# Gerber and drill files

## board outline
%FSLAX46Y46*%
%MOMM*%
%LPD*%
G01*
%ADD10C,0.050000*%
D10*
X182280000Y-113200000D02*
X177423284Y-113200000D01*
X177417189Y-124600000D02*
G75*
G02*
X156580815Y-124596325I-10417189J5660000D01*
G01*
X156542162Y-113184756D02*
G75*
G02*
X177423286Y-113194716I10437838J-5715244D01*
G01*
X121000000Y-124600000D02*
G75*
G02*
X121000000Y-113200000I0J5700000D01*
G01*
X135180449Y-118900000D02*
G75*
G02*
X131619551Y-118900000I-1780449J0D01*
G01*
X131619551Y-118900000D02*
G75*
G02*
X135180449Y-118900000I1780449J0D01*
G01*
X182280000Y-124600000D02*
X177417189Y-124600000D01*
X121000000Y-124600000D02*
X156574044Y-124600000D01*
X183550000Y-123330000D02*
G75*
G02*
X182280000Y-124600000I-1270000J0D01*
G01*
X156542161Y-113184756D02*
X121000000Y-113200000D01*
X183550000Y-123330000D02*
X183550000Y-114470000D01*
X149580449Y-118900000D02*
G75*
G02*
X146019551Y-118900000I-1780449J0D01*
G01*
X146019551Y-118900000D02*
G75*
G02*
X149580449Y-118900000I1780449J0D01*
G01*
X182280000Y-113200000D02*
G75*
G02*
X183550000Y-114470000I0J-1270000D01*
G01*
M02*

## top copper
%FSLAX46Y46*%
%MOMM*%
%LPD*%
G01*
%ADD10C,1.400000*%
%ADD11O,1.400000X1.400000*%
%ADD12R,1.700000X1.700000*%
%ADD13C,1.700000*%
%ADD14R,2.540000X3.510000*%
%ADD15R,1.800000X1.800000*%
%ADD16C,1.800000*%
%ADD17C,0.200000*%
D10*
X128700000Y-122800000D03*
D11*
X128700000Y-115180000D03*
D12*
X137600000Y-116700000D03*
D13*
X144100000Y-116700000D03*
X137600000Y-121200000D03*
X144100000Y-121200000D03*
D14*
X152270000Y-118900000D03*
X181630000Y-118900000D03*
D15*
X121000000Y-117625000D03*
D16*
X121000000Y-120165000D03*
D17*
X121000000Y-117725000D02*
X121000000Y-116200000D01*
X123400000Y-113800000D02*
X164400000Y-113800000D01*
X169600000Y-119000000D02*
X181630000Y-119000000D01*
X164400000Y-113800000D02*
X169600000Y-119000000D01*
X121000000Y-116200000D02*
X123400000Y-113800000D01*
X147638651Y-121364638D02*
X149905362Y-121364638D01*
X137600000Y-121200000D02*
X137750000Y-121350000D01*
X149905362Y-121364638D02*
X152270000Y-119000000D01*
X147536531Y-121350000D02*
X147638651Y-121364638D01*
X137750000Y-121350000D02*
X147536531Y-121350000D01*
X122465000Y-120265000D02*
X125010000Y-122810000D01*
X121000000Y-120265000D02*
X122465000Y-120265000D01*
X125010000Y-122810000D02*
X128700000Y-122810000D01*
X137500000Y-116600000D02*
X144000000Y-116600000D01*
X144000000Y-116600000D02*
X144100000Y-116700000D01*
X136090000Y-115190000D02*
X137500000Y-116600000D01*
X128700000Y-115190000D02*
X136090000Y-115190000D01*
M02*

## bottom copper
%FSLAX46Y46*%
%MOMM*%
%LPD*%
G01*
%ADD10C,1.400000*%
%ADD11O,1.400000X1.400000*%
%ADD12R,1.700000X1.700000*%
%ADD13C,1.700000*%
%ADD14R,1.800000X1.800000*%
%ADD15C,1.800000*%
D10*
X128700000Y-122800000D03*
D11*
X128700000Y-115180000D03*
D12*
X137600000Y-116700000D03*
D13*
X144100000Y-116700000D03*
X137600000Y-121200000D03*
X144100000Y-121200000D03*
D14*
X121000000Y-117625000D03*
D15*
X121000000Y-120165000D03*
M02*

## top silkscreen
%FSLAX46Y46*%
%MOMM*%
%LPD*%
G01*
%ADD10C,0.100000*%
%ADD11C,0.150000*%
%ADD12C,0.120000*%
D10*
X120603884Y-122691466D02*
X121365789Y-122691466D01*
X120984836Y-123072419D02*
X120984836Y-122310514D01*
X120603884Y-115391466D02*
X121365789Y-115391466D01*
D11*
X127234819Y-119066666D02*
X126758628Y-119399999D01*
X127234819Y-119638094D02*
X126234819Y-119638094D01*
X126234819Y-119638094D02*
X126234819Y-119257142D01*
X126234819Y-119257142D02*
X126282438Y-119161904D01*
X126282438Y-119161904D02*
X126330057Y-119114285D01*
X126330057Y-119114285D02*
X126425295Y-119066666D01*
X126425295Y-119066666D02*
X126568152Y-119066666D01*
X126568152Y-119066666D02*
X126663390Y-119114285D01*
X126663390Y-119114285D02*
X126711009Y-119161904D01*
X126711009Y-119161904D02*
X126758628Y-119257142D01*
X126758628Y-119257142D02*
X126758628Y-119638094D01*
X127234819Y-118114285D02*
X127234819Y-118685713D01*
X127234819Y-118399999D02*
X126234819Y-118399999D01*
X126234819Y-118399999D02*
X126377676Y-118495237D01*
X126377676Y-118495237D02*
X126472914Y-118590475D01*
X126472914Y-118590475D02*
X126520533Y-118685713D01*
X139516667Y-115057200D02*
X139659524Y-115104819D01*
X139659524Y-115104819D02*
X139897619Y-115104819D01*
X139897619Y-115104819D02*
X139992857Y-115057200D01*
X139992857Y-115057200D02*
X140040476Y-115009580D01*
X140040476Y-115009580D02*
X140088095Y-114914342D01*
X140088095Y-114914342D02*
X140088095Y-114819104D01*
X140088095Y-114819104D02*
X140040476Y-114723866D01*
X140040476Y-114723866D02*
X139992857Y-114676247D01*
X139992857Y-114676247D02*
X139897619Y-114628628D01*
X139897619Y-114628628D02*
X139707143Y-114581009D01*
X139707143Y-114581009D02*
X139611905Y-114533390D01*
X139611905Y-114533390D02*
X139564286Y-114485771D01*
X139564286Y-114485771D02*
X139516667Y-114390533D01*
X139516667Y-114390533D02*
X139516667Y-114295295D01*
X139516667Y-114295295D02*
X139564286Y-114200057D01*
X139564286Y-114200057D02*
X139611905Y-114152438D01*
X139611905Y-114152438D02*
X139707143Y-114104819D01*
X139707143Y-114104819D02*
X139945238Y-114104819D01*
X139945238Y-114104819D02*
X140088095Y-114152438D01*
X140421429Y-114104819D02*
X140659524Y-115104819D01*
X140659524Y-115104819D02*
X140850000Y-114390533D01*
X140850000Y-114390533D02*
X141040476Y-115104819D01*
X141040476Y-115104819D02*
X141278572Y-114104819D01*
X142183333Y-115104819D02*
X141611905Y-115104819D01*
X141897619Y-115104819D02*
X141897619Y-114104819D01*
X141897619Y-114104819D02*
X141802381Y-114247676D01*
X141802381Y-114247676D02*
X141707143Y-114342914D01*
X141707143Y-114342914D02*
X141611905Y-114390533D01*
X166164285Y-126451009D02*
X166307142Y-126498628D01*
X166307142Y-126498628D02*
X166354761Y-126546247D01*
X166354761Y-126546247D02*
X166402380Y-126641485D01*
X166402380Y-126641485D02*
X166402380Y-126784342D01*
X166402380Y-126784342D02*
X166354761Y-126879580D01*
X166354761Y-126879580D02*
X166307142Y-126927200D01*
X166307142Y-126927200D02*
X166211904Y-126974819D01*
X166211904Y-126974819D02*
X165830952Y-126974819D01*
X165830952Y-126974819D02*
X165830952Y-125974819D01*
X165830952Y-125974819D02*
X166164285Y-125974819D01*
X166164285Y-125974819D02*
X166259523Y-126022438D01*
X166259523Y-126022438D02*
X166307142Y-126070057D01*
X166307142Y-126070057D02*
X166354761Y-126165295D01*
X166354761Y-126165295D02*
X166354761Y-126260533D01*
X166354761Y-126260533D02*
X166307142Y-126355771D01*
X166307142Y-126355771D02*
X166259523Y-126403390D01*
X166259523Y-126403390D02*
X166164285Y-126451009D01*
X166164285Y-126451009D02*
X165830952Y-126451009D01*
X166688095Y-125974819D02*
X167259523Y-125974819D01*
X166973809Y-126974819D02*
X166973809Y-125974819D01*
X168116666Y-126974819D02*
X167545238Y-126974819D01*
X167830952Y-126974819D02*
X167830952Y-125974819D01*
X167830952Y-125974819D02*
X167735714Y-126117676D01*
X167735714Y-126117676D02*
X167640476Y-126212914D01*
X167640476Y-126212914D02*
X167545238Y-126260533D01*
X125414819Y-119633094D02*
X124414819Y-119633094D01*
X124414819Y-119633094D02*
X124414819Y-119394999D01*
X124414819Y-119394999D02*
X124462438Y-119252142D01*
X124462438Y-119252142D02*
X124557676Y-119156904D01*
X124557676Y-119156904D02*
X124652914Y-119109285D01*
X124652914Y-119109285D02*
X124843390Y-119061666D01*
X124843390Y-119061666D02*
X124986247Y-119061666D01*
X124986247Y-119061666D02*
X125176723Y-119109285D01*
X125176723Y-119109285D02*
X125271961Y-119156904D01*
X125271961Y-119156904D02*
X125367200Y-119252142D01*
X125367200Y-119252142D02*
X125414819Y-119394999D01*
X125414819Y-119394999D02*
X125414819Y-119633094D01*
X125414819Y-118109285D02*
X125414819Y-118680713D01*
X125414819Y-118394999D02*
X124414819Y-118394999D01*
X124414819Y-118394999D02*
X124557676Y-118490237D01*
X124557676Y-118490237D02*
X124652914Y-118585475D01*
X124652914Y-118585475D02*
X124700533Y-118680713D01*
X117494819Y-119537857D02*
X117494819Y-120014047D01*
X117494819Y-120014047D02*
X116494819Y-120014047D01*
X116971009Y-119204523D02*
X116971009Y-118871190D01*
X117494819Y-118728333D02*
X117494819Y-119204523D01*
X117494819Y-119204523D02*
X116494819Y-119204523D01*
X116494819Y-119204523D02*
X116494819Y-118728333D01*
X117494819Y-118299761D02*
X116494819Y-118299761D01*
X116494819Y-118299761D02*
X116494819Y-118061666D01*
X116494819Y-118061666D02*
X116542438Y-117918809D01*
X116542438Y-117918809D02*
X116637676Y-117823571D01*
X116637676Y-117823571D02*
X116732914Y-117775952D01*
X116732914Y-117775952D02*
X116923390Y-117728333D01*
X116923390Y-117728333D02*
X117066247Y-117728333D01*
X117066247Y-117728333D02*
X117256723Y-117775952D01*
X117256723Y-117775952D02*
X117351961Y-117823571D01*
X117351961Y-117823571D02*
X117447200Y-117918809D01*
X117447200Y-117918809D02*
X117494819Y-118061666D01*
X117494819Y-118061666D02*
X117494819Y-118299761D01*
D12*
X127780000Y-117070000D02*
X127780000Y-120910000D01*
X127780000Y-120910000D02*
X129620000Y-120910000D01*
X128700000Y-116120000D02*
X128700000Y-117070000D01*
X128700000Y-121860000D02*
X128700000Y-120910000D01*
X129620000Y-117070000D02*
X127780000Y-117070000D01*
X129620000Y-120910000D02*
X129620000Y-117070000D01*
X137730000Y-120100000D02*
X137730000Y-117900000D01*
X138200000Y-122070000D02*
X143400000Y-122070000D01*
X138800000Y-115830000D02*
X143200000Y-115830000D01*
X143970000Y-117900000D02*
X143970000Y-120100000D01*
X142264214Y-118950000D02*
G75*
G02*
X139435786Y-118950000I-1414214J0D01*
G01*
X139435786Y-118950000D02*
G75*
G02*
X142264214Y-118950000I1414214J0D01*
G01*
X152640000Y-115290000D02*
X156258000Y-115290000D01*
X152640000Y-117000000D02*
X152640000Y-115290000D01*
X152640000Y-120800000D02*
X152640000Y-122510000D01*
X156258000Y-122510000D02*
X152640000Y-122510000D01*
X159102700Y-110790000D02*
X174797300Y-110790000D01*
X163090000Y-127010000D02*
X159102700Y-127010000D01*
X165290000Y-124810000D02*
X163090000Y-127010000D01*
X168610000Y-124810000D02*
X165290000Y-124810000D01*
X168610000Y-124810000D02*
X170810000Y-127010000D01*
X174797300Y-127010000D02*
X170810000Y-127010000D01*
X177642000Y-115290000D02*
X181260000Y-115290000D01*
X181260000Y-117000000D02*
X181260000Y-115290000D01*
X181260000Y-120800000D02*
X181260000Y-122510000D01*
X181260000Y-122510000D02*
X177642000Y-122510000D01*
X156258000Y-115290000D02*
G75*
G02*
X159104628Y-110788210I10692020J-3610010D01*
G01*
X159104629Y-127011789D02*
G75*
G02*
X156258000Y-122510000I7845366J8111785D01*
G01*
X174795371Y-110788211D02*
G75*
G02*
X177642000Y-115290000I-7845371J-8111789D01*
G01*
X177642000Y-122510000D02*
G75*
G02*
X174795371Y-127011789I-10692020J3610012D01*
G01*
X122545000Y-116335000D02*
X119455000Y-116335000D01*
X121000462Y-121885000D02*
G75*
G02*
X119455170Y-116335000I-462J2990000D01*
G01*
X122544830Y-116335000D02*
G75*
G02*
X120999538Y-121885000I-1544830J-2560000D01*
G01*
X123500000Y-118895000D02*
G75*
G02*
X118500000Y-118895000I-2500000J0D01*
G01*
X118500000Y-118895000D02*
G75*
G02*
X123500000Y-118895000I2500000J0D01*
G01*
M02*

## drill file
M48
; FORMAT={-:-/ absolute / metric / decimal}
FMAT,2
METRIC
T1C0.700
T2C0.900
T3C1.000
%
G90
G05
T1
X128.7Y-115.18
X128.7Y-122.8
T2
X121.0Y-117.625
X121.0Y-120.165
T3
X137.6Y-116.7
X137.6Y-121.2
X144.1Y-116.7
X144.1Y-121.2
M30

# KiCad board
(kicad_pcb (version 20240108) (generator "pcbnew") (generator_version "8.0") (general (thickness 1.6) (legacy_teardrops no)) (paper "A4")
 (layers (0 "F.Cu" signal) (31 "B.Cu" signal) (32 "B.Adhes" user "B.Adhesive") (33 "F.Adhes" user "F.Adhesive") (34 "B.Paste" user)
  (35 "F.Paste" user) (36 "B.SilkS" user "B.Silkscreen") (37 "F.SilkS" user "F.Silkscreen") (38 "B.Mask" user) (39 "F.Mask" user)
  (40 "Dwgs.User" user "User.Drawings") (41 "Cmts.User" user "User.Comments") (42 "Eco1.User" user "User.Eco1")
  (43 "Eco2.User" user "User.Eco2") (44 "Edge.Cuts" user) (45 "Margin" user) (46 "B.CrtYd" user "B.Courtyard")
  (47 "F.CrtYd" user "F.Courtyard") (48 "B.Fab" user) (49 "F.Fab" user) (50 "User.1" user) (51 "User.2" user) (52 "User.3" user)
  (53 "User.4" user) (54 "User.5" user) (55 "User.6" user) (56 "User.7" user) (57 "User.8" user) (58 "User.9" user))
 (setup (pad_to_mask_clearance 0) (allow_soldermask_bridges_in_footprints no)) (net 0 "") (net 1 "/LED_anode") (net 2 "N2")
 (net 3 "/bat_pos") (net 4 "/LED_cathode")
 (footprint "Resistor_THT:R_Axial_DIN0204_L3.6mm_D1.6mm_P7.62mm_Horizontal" (layer "F.Cu") (at 128.7 122.8 90)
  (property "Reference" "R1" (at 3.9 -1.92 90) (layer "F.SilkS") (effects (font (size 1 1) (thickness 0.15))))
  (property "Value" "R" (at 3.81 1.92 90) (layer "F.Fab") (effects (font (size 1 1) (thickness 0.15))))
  (fp_line (start 5.73 -0.92) (end 1.89 -0.92) (stroke (width 0.12) (type solid)) (layer "F.SilkS"))
  (fp_line (start 1.89 -0.92) (end 1.89 0.92) (stroke (width 0.12) (type solid)) (layer "F.SilkS"))
  (fp_line (start 6.68 0) (end 5.73 0) (stroke (width 0.12) (type solid)) (layer "F.SilkS"))
  (fp_line (start 0.94 0) (end 1.89 0) (stroke (width 0.12) (type solid)) (layer "F.SilkS"))
  (fp_line (start 5.73 0.92) (end 5.73 -0.92) (stroke (width 0.12) (type solid)) (layer "F.SilkS"))
  (fp_line (start 1.89 0.92) (end 5.73 0.92) (stroke (width 0.12) (type solid)) (layer "F.SilkS"))
  (pad "1" thru_hole circle (at 0 0 90) (size 1.4 1.4) (drill 0.7) (layers "*.Cu" "*.Mask") (remove_unused_layers no) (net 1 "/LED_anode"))
  (pad "2" thru_hole oval (at 7.62 0 90) (size 1.4 1.4) (drill 0.7) (layers "*.Cu" "*.Mask") (remove_unused_layers no) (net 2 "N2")))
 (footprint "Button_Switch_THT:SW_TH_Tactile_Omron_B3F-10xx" (layer "F.Cu") (at 137.6 116.7)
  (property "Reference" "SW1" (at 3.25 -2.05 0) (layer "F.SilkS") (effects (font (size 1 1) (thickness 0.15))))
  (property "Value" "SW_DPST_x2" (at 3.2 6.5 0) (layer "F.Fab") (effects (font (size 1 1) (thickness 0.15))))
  (fp_line (start 0.13 3.4) (end 0.13 1.2) (stroke (width 0.12) (type solid)) (layer "F.SilkS"))
  (fp_line (start 0.6 5.37) (end 5.8 5.37) (stroke (width 0.12) (type solid)) (layer "F.SilkS"))
  (fp_line (start 1.2 -0.87) (end 5.6 -0.87) (stroke (width 0.12) (type solid)) (layer "F.SilkS"))
  (fp_line (start 6.37 1.2) (end 6.37 3.4) (stroke (width 0.12) (type solid)) (layer "F.SilkS"))
  (fp_circle (center 3.25 2.25) (end 4.25 3.25) (stroke (width 0.12) (type solid)) (fill none) (layer "F.SilkS"))
  (pad "1" thru_hole rect (at 0 0) (size 1.7 1.7) (drill 1) (layers "*.Cu" "*.Mask") (remove_unused_layers no) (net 2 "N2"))
  (pad "1" thru_hole circle (at 6.5 0) (size 1.7 1.7) (drill 1) (layers "*.Cu" "*.Mask") (remove_unused_layers no) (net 2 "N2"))
  (pad "2" thru_hole circle (at 0 4.5) (size 1.7 1.7) (drill 1) (layers "*.Cu" "*.Mask") (remove_unused_layers no) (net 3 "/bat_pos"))
  (pad "2" thru_hole circle (at 6.5 4.5) (size 1.7 1.7) (drill 1) (layers "*.Cu" "*.Mask") (remove_unused_layers no) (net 3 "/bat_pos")))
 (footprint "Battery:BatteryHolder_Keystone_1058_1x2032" (layer "F.Cu") (at 166.95 118.9)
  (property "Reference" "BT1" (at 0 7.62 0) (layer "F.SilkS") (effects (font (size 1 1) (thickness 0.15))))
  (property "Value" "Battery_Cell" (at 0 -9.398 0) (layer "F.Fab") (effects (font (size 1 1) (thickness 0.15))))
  (fp_line (start -14.31 -3.61) (end -10.692 -3.61) (stroke (width 0.12) (type solid)) (layer "F.SilkS"))
  (fp_line (start -14.31 -1.9) (end -14.31 -3.61) (stroke (width 0.12) (type solid)) (layer "F.SilkS"))
  (fp_line (start -14.31 1.9) (end -14.31 3.61) (stroke (width 0.12) (type solid)) (layer "F.SilkS"))
  (fp_line (start -10.692 3.61) (end -14.31 3.61) (stroke (width 0.12) (type solid)) (layer "F.SilkS"))
  (fp_line (start -7.8473 -8.11) (end 7.8473 -8.11) (stroke (width 0.12) (type solid)) (layer "F.SilkS"))
  (fp_line (start -3.86 8.11) (end -7.8473 8.11) (stroke (width 0.12) (type solid)) (layer "F.SilkS"))
  (fp_line (start -1.66 5.91) (end -3.86 8.11) (stroke (width 0.12) (type solid)) (layer "F.SilkS"))
  (fp_line (start 1.66 5.91) (end -1.66 5.91) (stroke (width 0.12) (type solid)) (layer "F.SilkS"))
  (fp_line (start 1.66 5.91) (end 3.86 8.11) (stroke (width 0.12) (type solid)) (layer "F.SilkS"))
  (fp_line (start 7.8473 8.11) (end 3.86 8.11) (stroke (width 0.12) (type solid)) (layer "F.SilkS"))
  (fp_line (start 10.692 -3.61) (end 14.31 -3.61) (stroke (width 0.12) (type solid)) (layer "F.SilkS"))
  (fp_line (start 14.31 -1.9) (end 14.31 -3.61) (stroke (width 0.12) (type solid)) (layer "F.SilkS"))
  (fp_line (start 14.31 1.9) (end 14.31 3.61) (stroke (width 0.12) (type solid)) (layer "F.SilkS"))
  (fp_line (start 14.31 3.61) (end 10.692 3.61) (stroke (width 0.12) (type solid)) (layer "F.SilkS"))
  (fp_arc (start -10.692 -3.61) (mid -9.538084 -6.031244) (end -7.845371 -8.111789) (stroke (width 0.12) (type solid)) (layer "F.SilkS"))
  (fp_arc (start -7.845371 8.111789) (mid -9.538085 6.031244) (end -10.692 3.61) (stroke (width 0.12) (type solid)) (layer "F.SilkS"))
  (fp_arc (start 7.845371 -8.111789) (mid 9.538085 -6.031244) (end 10.692 -3.61) (stroke (width 0.12) (type solid)) (layer "F.SilkS"))
  (fp_arc (start 10.692 3.61) (mid 9.538084 6.031244) (end 7.845371 8.111789) (stroke (width 0.12) (type solid)) (layer "F.SilkS"))
  (pad "1" smd rect (at -14.68 0) (size 2.54 3.51) (layers "F.Cu" "F.Paste" "F.Mask") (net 3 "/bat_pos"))
  (pad "2" smd rect (at 14.68 0) (size 2.54 3.51) (layers "F.Cu" "F.Paste" "F.Mask") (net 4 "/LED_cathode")))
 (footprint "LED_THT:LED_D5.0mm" (layer "F.Cu") (at 121 117.625 -90)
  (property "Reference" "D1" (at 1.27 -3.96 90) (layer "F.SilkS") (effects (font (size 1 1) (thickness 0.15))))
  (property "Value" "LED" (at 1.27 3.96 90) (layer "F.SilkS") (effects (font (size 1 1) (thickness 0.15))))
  (fp_line (start -1.29 -1.545) (end -1.29 1.545) (stroke (width 0.12) (type solid)) (layer "F.SilkS"))
  (fp_arc (start 4.26 -0.000462) (mid 2.072002 2.880433) (end -1.29 1.54483) (stroke (width 0.12) (type solid)) (layer "F.SilkS"))
  (fp_arc (start -1.29 -1.54483) (mid 2.072002 -2.880433) (end 4.26 0.000462) (stroke (width 0.12) (type solid)) (layer "F.SilkS"))
  (fp_circle (center 1.27 0) (end 3.77 0) (stroke (width 0.12) (type solid)) (fill none) (layer "F.SilkS"))
  (pad "1" thru_hole rect (at 0 0 270) (size 1.8 1.8) (drill 0.9) (layers "*.Cu" "*.Mask") (remove_unused_layers no) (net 4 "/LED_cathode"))
  (pad "2" thru_hole circle (at 2.54 0 270) (size 1.8 1.8) (drill 0.9) (layers "*.Cu" "*.Mask") (remove_unused_layers no)
   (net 1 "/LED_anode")))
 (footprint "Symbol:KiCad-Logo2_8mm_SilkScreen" (layer "B.Cu") (at 167 118.6 180)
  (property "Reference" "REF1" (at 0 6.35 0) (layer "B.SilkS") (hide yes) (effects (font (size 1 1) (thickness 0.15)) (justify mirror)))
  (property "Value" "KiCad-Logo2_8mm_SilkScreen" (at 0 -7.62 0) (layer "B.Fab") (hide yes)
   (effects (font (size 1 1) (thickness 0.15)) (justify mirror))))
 (gr_line (start 182.28 113.2) (end 177.423284 113.2) (stroke (width 0.05) (type default)) (layer "Edge.Cuts"))
 (gr_arc (start 177.417189 124.6) (mid 166.997909 130.795523) (end 156.580815 124.596325) (stroke (width 0.05) (type default))
  (layer "Edge.Cuts"))
 (gr_arc (start 156.542162 113.184756) (mid 166.985676 106.999897) (end 177.423286 113.194716) (stroke (width 0.05) (type default))
  (layer "Edge.Cuts"))
 (gr_arc (start 121 124.6) (mid 115.3 118.9) (end 121 113.2) (stroke (width 0.05) (type default)) (layer "Edge.Cuts"))
 (gr_circle (center 133.4 118.9) (end 132 117.8) (stroke (width 0.05) (type default)) (fill none) (layer "Edge.Cuts"))
 (gr_line (start 182.28 124.6) (end 177.417189 124.6) (stroke (width 0.05) (type default)) (layer "Edge.Cuts"))
 (gr_line (start 121 124.6) (end 156.574044 124.6) (stroke (width 0.05) (type default)) (layer "Edge.Cuts"))
 (gr_arc (start 183.55 123.33) (mid 183.178026 124.228026) (end 182.28 124.6) (stroke (width 0.05) (type default)) (layer "Edge.Cuts"))
 (gr_line (start 156.542161 113.184756) (end 121 113.2) (stroke (width 0.05) (type default)) (layer "Edge.Cuts"))
 (gr_line (start 183.55 123.33) (end 183.55 114.47) (stroke (width 0.05) (type default)) (layer "Edge.Cuts"))
 (gr_circle (center 147.8 118.9) (end 146.4 117.8) (stroke (width 0.05) (type default)) (fill none) (layer "Edge.Cuts"))
 (gr_arc (start 182.28 113.2) (mid 183.178026 113.571974) (end 183.55 114.47) (stroke (width 0.05) (type default)) (layer "Edge.Cuts"))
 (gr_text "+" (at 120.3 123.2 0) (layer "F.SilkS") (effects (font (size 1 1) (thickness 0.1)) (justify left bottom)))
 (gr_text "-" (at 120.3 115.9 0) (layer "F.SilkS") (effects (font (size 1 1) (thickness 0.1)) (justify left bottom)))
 (segment (start 121 117.725) (end 121 116.2) (width 0.2) (layer "F.Cu") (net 4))
 (segment (start 123.4 113.8) (end 164.4 113.8) (width 0.2) (layer "F.Cu") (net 4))
 (segment (start 169.6 119) (end 181.63 119) (width 0.2) (layer "F.Cu") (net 4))
 (segment (start 164.4 113.8) (end 169.6 119) (width 0.2) (layer "F.Cu") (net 4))
 (segment (start 121 116.2) (end 123.4 113.8) (width 0.2) (layer "F.Cu") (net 4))
 (segment (start 147.638651 121.364638) (end 149.905362 121.364638) (width 0.2) (layer "F.Cu") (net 3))
 (segment (start 137.6 121.2) (end 137.75 121.35) (width 0.2) (layer "F.Cu") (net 3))
 (segment (start 149.905362 121.364638) (end 152.27 119) (width 0.2) (layer "F.Cu") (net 3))
 (segment (start 147.536531 121.35) (end 147.638651 121.364638) (width 0.2) (layer "F.Cu") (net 3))
 (segment (start 137.75 121.35) (end 147.536531 121.35) (width 0.2) (layer "F.Cu") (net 3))
 (segment (start 122.465 120.265) (end 125.01 122.81) (width 0.2) (layer "F.Cu") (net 1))
 (segment (start 121 120.265) (end 122.465 120.265) (width 0.2) (layer "F.Cu") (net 1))
 (segment (start 125.01 122.81) (end 128.7 122.81) (width 0.2) (layer "F.Cu") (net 1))
 (segment (start 137.5 116.6) (end 144 116.6) (width 0.2) (layer "F.Cu") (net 2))
 (segment (start 144 116.6) (end 144.1 116.7) (width 0.2) (layer "F.Cu") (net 2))
 (segment (start 136.09 115.19) (end 137.5 116.6) (width 0.2) (layer "F.Cu") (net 2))
 (segment (start 128.7 115.19) (end 136.09 115.19) (width 0.2) (layer "F.Cu") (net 2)))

